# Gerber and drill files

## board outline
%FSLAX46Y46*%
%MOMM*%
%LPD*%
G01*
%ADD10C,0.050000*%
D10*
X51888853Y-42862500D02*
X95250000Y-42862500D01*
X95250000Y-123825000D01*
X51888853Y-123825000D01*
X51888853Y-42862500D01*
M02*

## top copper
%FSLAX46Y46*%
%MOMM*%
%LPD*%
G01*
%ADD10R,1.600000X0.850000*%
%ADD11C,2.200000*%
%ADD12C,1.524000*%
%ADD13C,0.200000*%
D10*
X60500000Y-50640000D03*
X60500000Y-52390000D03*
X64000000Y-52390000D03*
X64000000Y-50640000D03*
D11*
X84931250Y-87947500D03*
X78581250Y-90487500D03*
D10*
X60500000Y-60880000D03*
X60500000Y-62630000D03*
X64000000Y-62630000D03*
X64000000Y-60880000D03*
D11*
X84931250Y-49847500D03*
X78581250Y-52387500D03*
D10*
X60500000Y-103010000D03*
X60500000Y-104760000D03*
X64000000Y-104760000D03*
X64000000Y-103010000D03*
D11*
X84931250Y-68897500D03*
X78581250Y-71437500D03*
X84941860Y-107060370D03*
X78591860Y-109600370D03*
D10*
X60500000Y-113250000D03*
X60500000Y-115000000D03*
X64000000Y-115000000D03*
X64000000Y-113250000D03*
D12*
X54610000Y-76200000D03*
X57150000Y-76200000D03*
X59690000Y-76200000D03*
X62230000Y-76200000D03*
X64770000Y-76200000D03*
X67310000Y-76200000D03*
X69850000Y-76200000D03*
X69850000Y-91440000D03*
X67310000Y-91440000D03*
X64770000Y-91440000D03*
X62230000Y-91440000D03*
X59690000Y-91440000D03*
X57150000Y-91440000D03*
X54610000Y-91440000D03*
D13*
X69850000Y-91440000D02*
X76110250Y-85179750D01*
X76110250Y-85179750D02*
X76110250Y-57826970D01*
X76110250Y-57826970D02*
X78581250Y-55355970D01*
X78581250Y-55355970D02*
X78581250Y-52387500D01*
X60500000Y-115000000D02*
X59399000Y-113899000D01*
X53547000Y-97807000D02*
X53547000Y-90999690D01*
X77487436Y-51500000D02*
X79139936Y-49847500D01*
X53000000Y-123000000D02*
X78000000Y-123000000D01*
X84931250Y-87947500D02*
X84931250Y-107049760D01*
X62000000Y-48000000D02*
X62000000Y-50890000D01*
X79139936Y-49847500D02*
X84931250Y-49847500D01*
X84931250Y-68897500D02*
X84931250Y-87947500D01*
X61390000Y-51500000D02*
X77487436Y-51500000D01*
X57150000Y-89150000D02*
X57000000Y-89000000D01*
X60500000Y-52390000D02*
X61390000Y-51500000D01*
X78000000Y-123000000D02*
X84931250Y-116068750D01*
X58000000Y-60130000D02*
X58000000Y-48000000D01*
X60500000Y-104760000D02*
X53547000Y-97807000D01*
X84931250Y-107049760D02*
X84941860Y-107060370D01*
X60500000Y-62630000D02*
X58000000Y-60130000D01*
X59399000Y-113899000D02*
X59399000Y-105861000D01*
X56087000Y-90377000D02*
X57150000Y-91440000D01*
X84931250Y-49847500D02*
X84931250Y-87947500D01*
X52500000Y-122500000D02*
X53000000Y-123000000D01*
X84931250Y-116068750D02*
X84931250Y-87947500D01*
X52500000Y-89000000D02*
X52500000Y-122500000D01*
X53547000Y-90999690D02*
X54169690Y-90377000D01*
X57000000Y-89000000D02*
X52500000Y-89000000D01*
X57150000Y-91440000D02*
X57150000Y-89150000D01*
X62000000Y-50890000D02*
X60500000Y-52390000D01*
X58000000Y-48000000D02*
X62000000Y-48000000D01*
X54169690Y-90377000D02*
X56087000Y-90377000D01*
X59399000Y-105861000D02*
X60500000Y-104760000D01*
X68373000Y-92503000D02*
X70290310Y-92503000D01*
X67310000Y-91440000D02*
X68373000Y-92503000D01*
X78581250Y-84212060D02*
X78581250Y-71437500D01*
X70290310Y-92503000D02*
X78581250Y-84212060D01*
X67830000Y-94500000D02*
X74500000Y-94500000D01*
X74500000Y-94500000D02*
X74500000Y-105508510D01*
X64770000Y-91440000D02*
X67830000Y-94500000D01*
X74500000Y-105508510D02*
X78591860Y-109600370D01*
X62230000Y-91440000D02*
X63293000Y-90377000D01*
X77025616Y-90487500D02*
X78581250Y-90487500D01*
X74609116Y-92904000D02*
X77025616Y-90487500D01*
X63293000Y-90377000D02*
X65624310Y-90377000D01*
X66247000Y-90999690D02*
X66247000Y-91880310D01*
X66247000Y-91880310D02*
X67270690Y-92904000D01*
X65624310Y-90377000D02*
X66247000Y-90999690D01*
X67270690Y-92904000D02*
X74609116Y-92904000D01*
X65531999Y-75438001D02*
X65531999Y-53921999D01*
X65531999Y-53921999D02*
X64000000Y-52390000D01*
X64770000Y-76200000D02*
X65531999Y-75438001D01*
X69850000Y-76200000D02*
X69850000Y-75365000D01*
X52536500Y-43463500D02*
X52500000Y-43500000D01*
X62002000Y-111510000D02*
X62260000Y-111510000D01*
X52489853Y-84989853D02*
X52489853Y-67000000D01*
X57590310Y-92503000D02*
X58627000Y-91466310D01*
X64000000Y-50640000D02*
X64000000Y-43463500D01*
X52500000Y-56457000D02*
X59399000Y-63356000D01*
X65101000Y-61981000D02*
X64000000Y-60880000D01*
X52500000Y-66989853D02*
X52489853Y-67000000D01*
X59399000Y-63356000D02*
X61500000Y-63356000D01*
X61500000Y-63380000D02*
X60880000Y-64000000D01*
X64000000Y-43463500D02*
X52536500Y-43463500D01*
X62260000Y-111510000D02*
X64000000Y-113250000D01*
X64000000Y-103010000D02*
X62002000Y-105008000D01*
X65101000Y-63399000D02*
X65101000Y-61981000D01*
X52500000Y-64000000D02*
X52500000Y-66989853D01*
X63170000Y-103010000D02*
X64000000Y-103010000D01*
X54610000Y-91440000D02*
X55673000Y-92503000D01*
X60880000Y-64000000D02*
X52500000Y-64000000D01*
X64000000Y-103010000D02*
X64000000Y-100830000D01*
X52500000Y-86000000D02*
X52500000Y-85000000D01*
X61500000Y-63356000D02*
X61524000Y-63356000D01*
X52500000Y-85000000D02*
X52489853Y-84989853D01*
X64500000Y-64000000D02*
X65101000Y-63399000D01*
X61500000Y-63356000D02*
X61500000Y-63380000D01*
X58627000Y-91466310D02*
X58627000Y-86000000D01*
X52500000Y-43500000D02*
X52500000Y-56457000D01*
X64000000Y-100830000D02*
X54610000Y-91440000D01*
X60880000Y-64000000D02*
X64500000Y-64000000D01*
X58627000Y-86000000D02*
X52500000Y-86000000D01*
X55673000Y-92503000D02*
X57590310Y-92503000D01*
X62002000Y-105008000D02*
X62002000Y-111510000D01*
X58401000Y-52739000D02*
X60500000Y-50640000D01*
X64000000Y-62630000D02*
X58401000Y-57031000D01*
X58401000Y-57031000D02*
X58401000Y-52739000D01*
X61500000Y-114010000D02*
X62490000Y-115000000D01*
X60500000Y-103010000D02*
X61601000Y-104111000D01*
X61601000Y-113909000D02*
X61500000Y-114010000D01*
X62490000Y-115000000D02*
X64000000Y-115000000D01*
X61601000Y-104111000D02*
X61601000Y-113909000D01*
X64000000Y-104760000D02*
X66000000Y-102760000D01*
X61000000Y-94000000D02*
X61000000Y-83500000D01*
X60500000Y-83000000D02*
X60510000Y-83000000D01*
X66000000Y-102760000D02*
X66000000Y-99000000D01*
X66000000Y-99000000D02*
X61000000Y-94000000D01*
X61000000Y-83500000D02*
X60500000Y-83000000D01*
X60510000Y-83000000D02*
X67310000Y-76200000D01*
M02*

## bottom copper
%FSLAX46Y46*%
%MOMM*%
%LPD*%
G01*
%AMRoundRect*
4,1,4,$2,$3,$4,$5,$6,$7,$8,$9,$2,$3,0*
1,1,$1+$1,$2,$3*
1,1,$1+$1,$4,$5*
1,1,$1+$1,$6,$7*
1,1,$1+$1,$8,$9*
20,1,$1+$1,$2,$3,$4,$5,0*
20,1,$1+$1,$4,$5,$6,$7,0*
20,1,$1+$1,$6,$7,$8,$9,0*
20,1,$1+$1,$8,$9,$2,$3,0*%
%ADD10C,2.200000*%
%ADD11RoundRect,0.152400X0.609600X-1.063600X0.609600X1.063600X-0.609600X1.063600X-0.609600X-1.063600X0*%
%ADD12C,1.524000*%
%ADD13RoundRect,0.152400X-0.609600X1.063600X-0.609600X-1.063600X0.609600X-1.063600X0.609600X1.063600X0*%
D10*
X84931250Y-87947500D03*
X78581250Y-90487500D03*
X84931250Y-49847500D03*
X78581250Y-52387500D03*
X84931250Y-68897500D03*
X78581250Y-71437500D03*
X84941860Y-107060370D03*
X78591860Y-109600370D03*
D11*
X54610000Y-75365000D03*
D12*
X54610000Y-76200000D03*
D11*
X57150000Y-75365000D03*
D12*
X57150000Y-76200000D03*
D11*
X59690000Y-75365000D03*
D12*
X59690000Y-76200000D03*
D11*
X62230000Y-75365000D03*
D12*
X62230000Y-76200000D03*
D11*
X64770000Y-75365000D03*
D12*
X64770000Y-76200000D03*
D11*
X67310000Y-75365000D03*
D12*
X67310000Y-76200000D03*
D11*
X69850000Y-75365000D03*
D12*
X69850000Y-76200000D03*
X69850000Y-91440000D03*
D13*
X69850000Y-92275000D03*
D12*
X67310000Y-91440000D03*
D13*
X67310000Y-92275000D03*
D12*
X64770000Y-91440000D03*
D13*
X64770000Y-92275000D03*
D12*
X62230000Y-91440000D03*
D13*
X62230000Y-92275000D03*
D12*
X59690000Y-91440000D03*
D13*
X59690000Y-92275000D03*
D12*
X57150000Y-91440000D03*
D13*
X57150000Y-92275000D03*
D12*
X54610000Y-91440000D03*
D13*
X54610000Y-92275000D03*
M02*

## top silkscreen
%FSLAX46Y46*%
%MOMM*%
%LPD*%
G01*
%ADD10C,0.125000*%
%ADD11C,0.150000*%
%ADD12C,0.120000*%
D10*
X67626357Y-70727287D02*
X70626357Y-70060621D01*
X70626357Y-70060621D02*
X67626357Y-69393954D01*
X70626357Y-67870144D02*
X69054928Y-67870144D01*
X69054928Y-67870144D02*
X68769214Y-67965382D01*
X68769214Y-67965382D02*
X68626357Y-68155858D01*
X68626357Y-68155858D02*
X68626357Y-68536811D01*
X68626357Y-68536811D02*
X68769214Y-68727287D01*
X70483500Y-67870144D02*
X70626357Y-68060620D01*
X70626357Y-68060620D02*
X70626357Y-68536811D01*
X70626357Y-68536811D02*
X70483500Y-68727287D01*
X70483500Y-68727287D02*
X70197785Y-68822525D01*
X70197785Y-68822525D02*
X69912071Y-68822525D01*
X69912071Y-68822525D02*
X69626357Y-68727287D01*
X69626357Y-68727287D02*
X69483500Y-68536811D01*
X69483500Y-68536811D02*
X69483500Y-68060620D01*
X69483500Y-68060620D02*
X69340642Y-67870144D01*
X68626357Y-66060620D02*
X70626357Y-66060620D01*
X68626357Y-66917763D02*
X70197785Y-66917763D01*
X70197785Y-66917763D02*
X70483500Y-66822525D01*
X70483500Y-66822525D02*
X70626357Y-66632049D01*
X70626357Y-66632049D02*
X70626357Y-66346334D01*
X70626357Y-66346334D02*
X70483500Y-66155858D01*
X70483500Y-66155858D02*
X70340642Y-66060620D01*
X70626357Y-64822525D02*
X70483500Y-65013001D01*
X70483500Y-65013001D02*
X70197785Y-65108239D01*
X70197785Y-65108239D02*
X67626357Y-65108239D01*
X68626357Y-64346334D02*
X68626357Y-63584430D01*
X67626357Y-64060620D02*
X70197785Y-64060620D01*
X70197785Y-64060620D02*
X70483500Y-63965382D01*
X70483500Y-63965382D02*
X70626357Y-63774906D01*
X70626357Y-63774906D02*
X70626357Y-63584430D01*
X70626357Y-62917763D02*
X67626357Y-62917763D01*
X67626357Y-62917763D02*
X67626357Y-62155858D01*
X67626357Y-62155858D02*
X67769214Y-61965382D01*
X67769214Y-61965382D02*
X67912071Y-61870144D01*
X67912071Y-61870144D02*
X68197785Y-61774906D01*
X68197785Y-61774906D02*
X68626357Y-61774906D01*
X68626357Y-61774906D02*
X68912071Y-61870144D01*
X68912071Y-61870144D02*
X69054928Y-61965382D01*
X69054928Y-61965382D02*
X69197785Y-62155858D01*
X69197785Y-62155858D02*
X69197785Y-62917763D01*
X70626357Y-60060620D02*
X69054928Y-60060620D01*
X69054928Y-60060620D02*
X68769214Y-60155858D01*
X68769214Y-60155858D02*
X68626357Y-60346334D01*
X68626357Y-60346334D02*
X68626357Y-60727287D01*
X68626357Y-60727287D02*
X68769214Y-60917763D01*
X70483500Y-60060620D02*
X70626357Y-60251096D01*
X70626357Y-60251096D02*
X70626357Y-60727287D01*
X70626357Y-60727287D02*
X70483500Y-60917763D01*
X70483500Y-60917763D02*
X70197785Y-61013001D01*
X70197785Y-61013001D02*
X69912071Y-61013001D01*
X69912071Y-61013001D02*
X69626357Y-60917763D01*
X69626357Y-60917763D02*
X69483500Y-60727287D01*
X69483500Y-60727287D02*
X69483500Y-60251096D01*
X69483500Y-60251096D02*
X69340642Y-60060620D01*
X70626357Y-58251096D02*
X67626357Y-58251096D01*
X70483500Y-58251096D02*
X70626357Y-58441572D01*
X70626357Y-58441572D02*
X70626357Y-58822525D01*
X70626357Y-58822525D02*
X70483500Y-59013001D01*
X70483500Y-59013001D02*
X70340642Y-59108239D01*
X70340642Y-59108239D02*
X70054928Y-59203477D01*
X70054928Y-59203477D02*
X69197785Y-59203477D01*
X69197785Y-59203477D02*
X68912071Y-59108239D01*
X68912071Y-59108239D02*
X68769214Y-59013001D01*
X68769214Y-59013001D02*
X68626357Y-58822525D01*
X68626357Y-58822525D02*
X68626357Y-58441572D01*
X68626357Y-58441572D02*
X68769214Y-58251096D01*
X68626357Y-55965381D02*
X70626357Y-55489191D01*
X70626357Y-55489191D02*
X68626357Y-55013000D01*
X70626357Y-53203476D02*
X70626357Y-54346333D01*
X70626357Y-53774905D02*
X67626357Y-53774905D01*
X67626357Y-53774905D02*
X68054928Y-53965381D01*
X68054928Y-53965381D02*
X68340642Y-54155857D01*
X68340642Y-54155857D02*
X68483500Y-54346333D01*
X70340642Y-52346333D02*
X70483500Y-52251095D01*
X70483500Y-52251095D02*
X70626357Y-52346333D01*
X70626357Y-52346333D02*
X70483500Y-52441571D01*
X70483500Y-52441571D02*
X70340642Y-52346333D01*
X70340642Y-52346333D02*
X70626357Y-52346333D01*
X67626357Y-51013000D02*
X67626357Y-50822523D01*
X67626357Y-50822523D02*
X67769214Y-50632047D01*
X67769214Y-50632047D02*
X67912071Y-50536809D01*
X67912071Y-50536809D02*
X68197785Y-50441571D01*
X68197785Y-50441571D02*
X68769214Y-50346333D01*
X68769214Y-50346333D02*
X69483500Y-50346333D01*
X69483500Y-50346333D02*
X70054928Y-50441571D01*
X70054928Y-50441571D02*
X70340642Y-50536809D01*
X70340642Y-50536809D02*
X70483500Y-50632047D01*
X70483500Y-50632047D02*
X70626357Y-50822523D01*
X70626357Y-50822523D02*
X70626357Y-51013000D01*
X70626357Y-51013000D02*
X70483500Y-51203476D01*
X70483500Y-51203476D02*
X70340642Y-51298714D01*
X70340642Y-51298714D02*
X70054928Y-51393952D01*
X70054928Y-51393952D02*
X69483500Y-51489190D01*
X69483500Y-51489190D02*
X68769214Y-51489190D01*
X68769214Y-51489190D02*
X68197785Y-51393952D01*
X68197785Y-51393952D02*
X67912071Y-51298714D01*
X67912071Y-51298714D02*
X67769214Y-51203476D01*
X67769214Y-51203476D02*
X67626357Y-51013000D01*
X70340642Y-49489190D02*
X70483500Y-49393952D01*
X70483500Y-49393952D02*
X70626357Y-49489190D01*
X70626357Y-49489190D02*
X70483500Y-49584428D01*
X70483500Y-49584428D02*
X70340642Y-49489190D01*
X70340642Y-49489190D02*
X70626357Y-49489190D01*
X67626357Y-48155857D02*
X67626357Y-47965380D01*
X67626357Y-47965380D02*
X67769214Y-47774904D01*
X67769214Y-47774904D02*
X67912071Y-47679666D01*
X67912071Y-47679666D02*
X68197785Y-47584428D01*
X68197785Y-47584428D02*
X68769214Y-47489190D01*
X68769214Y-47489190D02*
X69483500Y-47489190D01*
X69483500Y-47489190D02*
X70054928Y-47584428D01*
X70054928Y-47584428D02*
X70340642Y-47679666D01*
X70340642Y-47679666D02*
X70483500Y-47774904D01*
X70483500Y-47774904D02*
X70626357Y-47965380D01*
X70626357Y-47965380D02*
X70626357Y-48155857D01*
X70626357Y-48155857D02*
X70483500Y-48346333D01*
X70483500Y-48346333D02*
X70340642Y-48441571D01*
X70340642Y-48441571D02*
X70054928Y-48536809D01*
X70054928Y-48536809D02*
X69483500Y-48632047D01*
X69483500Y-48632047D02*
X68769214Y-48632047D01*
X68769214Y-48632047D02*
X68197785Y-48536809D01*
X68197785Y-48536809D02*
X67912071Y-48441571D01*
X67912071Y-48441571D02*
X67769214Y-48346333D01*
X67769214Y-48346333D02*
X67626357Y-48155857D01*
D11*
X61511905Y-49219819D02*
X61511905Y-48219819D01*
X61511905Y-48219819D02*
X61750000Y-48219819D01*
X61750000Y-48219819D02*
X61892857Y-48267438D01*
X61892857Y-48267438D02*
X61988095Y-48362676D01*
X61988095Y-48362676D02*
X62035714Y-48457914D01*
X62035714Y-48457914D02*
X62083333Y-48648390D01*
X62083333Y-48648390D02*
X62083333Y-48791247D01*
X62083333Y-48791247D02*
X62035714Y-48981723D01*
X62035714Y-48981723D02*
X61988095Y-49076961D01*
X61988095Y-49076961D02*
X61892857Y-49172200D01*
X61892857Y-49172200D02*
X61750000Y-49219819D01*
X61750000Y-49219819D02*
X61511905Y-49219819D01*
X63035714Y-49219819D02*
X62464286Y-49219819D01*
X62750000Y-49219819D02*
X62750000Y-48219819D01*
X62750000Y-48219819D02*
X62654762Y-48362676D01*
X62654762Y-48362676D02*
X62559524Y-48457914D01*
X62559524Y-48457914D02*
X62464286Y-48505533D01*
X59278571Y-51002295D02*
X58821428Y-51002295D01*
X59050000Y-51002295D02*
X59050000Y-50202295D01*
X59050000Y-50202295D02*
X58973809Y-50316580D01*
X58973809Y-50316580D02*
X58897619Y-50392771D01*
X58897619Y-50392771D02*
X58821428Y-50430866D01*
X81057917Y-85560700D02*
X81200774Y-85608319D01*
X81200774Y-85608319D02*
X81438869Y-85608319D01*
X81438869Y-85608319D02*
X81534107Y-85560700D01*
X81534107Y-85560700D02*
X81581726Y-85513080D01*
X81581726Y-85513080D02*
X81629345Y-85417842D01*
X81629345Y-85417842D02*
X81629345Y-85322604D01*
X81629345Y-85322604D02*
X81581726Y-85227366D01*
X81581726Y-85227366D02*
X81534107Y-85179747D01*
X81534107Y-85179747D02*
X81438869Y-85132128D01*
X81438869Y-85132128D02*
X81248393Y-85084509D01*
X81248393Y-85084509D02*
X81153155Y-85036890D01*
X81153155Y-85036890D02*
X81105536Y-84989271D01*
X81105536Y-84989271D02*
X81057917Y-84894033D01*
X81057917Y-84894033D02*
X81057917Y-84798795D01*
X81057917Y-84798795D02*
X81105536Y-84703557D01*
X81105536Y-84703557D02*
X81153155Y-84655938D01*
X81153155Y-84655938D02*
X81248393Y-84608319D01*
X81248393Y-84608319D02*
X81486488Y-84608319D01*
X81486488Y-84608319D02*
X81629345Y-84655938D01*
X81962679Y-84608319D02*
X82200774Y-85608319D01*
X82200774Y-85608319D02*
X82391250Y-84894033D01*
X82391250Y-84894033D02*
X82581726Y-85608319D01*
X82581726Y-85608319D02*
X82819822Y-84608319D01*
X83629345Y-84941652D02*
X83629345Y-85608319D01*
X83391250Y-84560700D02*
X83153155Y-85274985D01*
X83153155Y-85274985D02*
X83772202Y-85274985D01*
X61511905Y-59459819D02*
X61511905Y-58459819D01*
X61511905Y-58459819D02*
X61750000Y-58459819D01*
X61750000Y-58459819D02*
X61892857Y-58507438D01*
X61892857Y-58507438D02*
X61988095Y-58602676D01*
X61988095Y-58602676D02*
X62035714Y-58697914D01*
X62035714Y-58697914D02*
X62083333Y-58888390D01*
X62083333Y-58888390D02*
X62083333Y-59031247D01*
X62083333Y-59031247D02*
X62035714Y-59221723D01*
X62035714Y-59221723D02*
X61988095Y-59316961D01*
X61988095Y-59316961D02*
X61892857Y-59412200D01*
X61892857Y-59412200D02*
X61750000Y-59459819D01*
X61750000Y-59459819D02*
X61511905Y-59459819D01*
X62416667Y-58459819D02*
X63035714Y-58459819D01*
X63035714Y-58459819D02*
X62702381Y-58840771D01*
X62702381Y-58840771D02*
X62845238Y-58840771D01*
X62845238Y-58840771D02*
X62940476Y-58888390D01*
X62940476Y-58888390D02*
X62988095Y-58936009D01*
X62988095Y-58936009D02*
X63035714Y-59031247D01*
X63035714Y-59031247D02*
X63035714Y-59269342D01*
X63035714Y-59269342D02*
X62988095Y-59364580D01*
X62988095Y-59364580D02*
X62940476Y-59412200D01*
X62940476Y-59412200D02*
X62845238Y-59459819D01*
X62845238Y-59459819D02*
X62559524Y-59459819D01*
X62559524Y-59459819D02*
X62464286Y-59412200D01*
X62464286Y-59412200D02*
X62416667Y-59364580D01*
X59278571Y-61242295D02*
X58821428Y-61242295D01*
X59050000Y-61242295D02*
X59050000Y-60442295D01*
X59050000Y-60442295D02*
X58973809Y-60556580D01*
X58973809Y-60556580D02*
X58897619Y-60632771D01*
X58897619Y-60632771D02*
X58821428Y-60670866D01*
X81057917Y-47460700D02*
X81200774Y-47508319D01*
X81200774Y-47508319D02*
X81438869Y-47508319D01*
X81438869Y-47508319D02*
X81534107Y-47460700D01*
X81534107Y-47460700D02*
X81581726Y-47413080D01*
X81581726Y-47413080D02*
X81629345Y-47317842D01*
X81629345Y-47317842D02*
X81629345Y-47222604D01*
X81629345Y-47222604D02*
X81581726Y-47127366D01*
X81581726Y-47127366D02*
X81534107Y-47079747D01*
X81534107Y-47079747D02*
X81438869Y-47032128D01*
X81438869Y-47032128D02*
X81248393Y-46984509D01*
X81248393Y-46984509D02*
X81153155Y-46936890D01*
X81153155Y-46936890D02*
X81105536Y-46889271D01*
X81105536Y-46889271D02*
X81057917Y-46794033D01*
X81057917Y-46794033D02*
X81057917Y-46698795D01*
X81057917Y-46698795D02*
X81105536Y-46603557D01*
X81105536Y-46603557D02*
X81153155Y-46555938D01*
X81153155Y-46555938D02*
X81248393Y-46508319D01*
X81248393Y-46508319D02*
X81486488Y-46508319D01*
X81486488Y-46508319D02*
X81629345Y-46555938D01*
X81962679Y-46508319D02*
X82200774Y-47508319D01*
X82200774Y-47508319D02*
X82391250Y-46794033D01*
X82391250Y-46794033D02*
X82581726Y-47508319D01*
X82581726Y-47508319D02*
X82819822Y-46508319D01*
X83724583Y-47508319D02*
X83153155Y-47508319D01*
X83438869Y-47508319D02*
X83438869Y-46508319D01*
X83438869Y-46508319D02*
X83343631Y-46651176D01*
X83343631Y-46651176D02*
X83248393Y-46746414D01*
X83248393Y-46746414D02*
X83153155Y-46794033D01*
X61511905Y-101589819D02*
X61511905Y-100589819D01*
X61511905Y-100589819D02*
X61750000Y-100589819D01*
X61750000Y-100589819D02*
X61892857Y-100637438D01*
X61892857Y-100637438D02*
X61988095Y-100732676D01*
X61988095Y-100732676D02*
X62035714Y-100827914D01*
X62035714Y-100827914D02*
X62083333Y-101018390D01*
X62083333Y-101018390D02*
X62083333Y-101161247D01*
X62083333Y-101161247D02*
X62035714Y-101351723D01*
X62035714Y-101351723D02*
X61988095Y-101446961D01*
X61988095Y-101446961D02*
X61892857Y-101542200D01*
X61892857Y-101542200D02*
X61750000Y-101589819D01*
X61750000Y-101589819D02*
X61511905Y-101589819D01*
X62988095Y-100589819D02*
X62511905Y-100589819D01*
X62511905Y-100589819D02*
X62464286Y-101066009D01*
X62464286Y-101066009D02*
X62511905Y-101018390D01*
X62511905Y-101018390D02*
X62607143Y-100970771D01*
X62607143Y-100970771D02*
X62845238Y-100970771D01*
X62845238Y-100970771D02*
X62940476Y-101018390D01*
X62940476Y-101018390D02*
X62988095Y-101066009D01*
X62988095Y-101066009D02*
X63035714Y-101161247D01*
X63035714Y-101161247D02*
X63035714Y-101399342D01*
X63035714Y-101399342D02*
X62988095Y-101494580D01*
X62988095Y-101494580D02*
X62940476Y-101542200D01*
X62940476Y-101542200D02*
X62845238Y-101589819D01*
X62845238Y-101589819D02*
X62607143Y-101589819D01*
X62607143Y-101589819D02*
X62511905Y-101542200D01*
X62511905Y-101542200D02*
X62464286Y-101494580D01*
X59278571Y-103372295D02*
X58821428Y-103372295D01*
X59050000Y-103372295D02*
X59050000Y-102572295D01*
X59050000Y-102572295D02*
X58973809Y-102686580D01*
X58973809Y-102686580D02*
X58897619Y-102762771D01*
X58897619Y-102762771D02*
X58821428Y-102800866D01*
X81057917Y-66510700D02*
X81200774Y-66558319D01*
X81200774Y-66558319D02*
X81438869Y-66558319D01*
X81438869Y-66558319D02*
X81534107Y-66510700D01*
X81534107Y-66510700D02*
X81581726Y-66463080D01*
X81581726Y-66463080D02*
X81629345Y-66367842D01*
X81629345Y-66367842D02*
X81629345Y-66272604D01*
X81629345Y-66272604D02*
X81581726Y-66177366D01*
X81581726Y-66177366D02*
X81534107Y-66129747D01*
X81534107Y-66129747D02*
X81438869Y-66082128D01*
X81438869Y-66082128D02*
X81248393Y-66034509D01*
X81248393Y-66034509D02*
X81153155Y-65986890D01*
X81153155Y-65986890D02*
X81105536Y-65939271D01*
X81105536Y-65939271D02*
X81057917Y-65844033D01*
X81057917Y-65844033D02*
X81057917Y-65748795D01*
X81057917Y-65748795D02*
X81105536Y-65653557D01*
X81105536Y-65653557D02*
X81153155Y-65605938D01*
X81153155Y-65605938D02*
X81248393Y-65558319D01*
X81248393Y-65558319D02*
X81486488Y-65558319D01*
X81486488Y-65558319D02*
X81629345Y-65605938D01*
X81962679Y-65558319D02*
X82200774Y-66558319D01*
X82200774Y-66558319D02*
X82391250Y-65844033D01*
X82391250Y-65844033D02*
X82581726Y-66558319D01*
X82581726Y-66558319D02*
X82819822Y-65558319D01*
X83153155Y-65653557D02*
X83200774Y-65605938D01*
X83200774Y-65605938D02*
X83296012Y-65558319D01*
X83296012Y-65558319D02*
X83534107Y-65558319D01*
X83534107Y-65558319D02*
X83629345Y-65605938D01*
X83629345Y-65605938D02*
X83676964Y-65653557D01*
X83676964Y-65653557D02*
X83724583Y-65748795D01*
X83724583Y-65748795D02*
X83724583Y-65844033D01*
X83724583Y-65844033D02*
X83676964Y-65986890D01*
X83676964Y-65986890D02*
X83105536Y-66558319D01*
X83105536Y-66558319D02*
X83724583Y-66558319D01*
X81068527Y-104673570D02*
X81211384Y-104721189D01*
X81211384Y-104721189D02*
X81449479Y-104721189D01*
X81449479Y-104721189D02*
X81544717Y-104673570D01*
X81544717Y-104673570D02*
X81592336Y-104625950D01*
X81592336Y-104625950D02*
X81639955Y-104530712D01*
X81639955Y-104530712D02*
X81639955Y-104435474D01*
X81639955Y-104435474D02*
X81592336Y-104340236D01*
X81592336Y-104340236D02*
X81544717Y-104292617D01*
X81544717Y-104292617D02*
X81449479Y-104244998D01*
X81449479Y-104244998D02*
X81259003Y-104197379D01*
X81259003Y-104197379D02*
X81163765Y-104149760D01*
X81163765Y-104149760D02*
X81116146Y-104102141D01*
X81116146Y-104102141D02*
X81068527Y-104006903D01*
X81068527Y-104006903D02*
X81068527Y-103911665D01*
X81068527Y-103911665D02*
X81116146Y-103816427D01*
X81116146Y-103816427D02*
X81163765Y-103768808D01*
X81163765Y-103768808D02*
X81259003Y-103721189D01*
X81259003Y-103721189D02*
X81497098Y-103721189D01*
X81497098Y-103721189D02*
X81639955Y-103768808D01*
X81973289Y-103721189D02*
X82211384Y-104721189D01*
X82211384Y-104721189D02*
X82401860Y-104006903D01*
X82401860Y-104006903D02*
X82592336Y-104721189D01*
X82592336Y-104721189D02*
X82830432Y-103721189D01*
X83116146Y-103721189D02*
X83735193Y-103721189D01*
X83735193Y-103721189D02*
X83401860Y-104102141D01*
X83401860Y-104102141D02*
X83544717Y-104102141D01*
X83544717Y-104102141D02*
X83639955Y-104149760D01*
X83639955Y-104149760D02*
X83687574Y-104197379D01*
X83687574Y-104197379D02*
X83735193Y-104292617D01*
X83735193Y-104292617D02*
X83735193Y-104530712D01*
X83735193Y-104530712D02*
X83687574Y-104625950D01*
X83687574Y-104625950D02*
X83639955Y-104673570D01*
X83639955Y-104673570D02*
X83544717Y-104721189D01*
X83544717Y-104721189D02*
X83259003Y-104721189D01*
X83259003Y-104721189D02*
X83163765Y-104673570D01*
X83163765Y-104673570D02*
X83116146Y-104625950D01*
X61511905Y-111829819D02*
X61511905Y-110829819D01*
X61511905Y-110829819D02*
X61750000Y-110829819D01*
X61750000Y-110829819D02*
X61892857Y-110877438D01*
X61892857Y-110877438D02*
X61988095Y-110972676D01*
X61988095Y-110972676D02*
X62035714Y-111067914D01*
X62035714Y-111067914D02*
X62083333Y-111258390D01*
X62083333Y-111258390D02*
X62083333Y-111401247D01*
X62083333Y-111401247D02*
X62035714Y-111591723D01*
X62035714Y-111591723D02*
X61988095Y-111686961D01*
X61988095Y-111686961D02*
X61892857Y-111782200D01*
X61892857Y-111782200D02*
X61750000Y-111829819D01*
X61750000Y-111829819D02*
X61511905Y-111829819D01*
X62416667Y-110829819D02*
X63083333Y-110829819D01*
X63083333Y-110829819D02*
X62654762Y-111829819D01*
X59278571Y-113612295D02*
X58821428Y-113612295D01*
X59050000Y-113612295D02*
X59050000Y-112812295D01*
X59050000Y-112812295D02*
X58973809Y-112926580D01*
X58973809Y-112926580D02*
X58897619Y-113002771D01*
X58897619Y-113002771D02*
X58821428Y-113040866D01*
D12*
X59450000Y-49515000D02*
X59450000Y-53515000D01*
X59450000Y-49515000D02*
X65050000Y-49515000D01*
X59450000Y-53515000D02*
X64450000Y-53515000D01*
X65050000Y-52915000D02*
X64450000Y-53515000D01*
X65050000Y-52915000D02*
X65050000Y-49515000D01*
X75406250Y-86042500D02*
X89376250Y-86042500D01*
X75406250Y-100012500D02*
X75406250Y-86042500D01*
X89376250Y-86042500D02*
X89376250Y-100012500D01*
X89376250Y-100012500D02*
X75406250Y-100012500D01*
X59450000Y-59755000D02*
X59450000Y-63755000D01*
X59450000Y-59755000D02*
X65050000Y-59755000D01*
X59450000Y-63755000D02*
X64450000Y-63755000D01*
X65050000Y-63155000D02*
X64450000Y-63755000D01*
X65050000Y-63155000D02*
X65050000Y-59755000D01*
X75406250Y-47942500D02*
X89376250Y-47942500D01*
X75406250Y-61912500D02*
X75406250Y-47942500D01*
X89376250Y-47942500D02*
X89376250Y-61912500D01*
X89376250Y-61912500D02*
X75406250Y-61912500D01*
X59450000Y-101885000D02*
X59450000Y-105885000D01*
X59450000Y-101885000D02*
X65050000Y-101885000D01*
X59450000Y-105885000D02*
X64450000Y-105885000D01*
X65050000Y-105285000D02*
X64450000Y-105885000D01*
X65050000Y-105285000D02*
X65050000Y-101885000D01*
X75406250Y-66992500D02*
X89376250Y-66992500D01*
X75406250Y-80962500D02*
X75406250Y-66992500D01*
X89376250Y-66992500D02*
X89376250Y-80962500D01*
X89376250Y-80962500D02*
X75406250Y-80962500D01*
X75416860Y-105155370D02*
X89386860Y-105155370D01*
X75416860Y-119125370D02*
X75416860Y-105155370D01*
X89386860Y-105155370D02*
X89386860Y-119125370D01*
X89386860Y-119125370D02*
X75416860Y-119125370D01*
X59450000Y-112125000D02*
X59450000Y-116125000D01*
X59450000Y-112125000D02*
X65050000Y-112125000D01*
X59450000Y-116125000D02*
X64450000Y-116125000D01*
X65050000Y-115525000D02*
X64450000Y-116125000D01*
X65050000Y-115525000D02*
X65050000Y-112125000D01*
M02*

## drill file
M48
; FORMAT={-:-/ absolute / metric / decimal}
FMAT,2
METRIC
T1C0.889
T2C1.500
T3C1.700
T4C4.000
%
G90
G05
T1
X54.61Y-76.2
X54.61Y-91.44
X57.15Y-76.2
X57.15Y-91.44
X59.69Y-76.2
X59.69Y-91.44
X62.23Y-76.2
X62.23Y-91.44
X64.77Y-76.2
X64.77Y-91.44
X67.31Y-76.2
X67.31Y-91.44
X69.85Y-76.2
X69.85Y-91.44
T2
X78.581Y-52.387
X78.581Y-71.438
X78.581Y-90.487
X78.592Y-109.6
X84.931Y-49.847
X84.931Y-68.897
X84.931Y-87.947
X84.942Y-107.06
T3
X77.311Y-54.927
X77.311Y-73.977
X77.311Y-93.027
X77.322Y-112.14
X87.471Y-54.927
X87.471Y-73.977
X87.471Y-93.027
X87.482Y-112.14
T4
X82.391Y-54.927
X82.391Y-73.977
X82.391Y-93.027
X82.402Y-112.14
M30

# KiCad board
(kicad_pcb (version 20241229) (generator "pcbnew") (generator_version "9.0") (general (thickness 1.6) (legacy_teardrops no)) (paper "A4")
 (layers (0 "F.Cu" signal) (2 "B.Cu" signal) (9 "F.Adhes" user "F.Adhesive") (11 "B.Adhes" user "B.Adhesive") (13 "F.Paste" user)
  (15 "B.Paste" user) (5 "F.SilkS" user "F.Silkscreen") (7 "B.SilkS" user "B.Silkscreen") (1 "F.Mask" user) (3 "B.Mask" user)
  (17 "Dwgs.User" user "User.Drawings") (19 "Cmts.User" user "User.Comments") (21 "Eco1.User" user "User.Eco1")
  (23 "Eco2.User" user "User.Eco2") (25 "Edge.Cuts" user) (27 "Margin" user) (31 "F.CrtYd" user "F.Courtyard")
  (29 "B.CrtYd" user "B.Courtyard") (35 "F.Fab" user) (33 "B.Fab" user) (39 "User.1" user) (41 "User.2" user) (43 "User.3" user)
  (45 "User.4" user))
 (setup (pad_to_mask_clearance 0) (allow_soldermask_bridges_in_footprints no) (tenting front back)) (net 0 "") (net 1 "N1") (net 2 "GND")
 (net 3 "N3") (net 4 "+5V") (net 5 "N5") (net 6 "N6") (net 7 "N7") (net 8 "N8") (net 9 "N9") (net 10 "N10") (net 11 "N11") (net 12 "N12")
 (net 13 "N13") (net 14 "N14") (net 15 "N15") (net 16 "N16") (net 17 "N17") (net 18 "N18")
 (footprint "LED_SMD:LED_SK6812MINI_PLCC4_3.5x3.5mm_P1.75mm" (layer "F.Cu") (at 62.25 51.515)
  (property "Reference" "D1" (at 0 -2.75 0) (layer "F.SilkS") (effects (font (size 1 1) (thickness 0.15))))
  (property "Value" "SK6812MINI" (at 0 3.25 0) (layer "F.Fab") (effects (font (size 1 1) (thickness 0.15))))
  (fp_line (start -2.8 -2) (end -2.8 2) (stroke (width 0.12) (type default)) (layer "F.SilkS"))
  (fp_line (start -2.8 -2) (end 2.8 -2) (stroke (width 0.12) (type solid)) (layer "F.SilkS"))
  (fp_line (start -2.8 2) (end 2.2 2) (stroke (width 0.12) (type solid)) (layer "F.SilkS"))
  (fp_line (start 2.8 1.4) (end 2.2 2) (stroke (width 0.12) (type default)) (layer "F.SilkS"))
  (fp_line (start 2.8 1.4) (end 2.8 -2) (stroke (width 0.12) (type solid)) (layer "F.SilkS"))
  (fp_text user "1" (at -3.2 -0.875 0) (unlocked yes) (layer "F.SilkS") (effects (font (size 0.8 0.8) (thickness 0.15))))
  (pad "1" smd rect (at -1.75 -0.875) (size 1.6 0.85) (layers "F.Cu" "F.Mask" "F.Paste") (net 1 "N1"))
  (pad "2" smd rect (at -1.75 0.875) (size 1.6 0.85) (layers "F.Cu" "F.Mask" "F.Paste") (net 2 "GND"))
  (pad "3" smd rect (at 1.75 0.875) (size 1.6 0.85) (layers "F.Cu" "F.Mask" "F.Paste") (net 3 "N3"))
  (pad "4" smd rect (at 1.75 -0.875) (size 1.6 0.85) (layers "F.Cu" "F.Mask" "F.Paste") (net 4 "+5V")))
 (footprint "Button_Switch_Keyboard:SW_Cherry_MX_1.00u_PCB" (layer "F.Cu") (at 84.93125 87.9475)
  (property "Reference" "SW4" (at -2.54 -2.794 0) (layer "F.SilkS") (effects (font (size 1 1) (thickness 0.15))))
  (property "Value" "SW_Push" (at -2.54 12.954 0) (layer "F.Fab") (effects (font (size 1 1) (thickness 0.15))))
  (fp_line (start -9.525 -1.905) (end 4.445 -1.905) (stroke (width 0.12) (type solid)) (layer "F.SilkS"))
  (fp_line (start -9.525 12.065) (end -9.525 -1.905) (stroke (width 0.12) (type solid)) (layer "F.SilkS"))
  (fp_line (start 4.445 -1.905) (end 4.445 12.065) (stroke (width 0.12) (type solid)) (layer "F.SilkS"))
  (fp_line (start 4.445 12.065) (end -9.525 12.065) (stroke (width 0.12) (type solid)) (layer "F.SilkS"))
  (pad "" np_thru_hole circle (at -7.62 5.08) (size 1.7 1.7) (drill 1.7) (layers "*.Cu" "*.Mask"))
  (pad "" np_thru_hole circle (at -2.54 5.08) (size 4 4) (drill 4) (layers "*.Cu" "*.Mask"))
  (pad "" np_thru_hole circle (at 2.54 5.08) (size 1.7 1.7) (drill 1.7) (layers "*.Cu" "*.Mask"))
  (pad "1" thru_hole circle (at 0 0) (size 2.2 2.2) (drill 1.5) (layers "*.Cu" "*.Mask") (remove_unused_layers no) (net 2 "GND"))
  (pad "2" thru_hole circle (at -6.35 2.54) (size 2.2 2.2) (drill 1.5) (layers "*.Cu" "*.Mask") (remove_unused_layers no) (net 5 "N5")))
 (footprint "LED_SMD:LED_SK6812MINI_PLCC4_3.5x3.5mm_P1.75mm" (layer "F.Cu") (at 62.25 61.755)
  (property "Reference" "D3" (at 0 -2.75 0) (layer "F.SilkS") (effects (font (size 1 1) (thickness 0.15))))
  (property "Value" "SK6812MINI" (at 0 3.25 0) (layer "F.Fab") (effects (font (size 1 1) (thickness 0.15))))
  (fp_line (start -2.8 -2) (end -2.8 2) (stroke (width 0.12) (type default)) (layer "F.SilkS"))
  (fp_line (start -2.8 -2) (end 2.8 -2) (stroke (width 0.12) (type solid)) (layer "F.SilkS"))
  (fp_line (start -2.8 2) (end 2.2 2) (stroke (width 0.12) (type solid)) (layer "F.SilkS"))
  (fp_line (start 2.8 1.4) (end 2.2 2) (stroke (width 0.12) (type default)) (layer "F.SilkS"))
  (fp_line (start 2.8 1.4) (end 2.8 -2) (stroke (width 0.12) (type solid)) (layer "F.SilkS"))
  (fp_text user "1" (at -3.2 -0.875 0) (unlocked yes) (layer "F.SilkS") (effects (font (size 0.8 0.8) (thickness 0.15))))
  (pad "1" smd rect (at -1.75 -0.875) (size 1.6 0.85) (layers "F.Cu" "F.Mask" "F.Paste") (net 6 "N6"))
  (pad "2" smd rect (at -1.75 0.875) (size 1.6 0.85) (layers "F.Cu" "F.Mask" "F.Paste") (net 2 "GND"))
  (pad "3" smd rect (at 1.75 0.875) (size 1.6 0.85) (layers "F.Cu" "F.Mask" "F.Paste") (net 1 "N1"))
  (pad "4" smd rect (at 1.75 -0.875) (size 1.6 0.85) (layers "F.Cu" "F.Mask" "F.Paste") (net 4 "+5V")))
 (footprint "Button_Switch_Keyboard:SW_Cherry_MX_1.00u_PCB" (layer "F.Cu") (at 84.93125 49.8475)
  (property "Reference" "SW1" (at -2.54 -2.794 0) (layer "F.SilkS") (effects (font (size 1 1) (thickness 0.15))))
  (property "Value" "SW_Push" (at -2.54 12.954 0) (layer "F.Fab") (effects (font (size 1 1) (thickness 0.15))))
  (fp_line (start -9.525 -1.905) (end 4.445 -1.905) (stroke (width 0.12) (type solid)) (layer "F.SilkS"))
  (fp_line (start -9.525 12.065) (end -9.525 -1.905) (stroke (width 0.12) (type solid)) (layer "F.SilkS"))
  (fp_line (start 4.445 -1.905) (end 4.445 12.065) (stroke (width 0.12) (type solid)) (layer "F.SilkS"))
  (fp_line (start 4.445 12.065) (end -9.525 12.065) (stroke (width 0.12) (type solid)) (layer "F.SilkS"))
  (pad "" np_thru_hole circle (at -7.62 5.08) (size 1.7 1.7) (drill 1.7) (layers "*.Cu" "*.Mask"))
  (pad "" np_thru_hole circle (at -2.54 5.08) (size 4 4) (drill 4) (layers "*.Cu" "*.Mask"))
  (pad "" np_thru_hole circle (at 2.54 5.08) (size 1.7 1.7) (drill 1.7) (layers "*.Cu" "*.Mask"))
  (pad "1" thru_hole circle (at 0 0) (size 2.2 2.2) (drill 1.5) (layers "*.Cu" "*.Mask") (remove_unused_layers no) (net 2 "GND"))
  (pad "2" thru_hole circle (at -6.35 2.54) (size 2.2 2.2) (drill 1.5) (layers "*.Cu" "*.Mask") (remove_unused_layers no) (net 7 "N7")))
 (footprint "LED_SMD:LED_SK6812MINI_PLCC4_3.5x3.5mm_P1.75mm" (layer "F.Cu") (at 62.25 103.885)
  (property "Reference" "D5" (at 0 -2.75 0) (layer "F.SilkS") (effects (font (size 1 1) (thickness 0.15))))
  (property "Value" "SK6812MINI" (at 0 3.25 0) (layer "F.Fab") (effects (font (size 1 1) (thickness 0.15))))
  (fp_line (start -2.8 -2) (end -2.8 2) (stroke (width 0.12) (type default)) (layer "F.SilkS"))
  (fp_line (start -2.8 -2) (end 2.8 -2) (stroke (width 0.12) (type solid)) (layer "F.SilkS"))
  (fp_line (start -2.8 2) (end 2.2 2) (stroke (width 0.12) (type solid)) (layer "F.SilkS"))
  (fp_line (start 2.8 1.4) (end 2.2 2) (stroke (width 0.12) (type default)) (layer "F.SilkS"))
  (fp_line (start 2.8 1.4) (end 2.8 -2) (stroke (width 0.12) (type solid)) (layer "F.SilkS"))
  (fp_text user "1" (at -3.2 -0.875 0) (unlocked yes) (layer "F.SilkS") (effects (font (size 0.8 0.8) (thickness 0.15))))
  (pad "1" smd rect (at -1.75 -0.875) (size 1.6 0.85) (layers "F.Cu" "F.Mask" "F.Paste") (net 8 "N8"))
  (pad "2" smd rect (at -1.75 0.875) (size 1.6 0.85) (layers "F.Cu" "F.Mask" "F.Paste") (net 2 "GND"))
  (pad "3" smd rect (at 1.75 0.875) (size 1.6 0.85) (layers "F.Cu" "F.Mask" "F.Paste") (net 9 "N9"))
  (pad "4" smd rect (at 1.75 -0.875) (size 1.6 0.85) (layers "F.Cu" "F.Mask" "F.Paste") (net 4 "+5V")))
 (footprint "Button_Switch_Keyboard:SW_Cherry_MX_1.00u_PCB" (layer "F.Cu") (at 84.93125 68.8975)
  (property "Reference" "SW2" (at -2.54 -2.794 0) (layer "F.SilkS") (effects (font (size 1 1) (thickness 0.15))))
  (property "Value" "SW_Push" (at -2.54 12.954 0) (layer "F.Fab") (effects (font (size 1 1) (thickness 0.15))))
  (fp_line (start -9.525 -1.905) (end 4.445 -1.905) (stroke (width 0.12) (type solid)) (layer "F.SilkS"))
  (fp_line (start -9.525 12.065) (end -9.525 -1.905) (stroke (width 0.12) (type solid)) (layer "F.SilkS"))
  (fp_line (start 4.445 -1.905) (end 4.445 12.065) (stroke (width 0.12) (type solid)) (layer "F.SilkS"))
  (fp_line (start 4.445 12.065) (end -9.525 12.065) (stroke (width 0.12) (type solid)) (layer "F.SilkS"))
  (pad "" np_thru_hole circle (at -7.62 5.08) (size 1.7 1.7) (drill 1.7) (layers "*.Cu" "*.Mask"))
  (pad "" np_thru_hole circle (at -2.54 5.08) (size 4 4) (drill 4) (layers "*.Cu" "*.Mask"))
  (pad "" np_thru_hole circle (at 2.54 5.08) (size 1.7 1.7) (drill 1.7) (layers "*.Cu" "*.Mask"))
  (pad "1" thru_hole circle (at 0 0) (size 2.2 2.2) (drill 1.5) (layers "*.Cu" "*.Mask") (remove_unused_layers no) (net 2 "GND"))
  (pad "2" thru_hole circle (at -6.35 2.54) (size 2.2 2.2) (drill 1.5) (layers "*.Cu" "*.Mask") (remove_unused_layers no) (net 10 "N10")))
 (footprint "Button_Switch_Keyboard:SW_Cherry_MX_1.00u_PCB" (layer "F.Cu") (at 84.94186 107.06037)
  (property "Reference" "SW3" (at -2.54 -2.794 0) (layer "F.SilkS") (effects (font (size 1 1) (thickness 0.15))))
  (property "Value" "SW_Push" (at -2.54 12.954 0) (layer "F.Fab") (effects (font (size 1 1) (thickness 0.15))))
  (fp_line (start -9.525 -1.905) (end 4.445 -1.905) (stroke (width 0.12) (type solid)) (layer "F.SilkS"))
  (fp_line (start -9.525 12.065) (end -9.525 -1.905) (stroke (width 0.12) (type solid)) (layer "F.SilkS"))
  (fp_line (start 4.445 -1.905) (end 4.445 12.065) (stroke (width 0.12) (type solid)) (layer "F.SilkS"))
  (fp_line (start 4.445 12.065) (end -9.525 12.065) (stroke (width 0.12) (type solid)) (layer "F.SilkS"))
  (pad "" np_thru_hole circle (at -7.62 5.08) (size 1.7 1.7) (drill 1.7) (layers "*.Cu" "*.Mask"))
  (pad "" np_thru_hole circle (at -2.54 5.08) (size 4 4) (drill 4) (layers "*.Cu" "*.Mask"))
  (pad "" np_thru_hole circle (at 2.54 5.08) (size 1.7 1.7) (drill 1.7) (layers "*.Cu" "*.Mask"))
  (pad "1" thru_hole circle (at 0 0) (size 2.2 2.2) (drill 1.5) (layers "*.Cu" "*.Mask") (remove_unused_layers no) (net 2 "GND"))
  (pad "2" thru_hole circle (at -6.35 2.54) (size 2.2 2.2) (drill 1.5) (layers "*.Cu" "*.Mask") (remove_unused_layers no) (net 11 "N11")))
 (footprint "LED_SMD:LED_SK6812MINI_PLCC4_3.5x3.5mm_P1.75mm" (layer "F.Cu") (at 62.25 114.125)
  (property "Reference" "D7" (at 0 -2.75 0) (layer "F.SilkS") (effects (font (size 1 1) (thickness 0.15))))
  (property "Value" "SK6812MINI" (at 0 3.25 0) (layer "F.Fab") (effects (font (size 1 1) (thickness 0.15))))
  (fp_line (start -2.8 -2) (end -2.8 2) (stroke (width 0.12) (type default)) (layer "F.SilkS"))
  (fp_line (start -2.8 -2) (end 2.8 -2) (stroke (width 0.12) (type solid)) (layer "F.SilkS"))
  (fp_line (start -2.8 2) (end 2.2 2) (stroke (width 0.12) (type solid)) (layer "F.SilkS"))
  (fp_line (start 2.8 1.4) (end 2.2 2) (stroke (width 0.12) (type default)) (layer "F.SilkS"))
  (fp_line (start 2.8 1.4) (end 2.8 -2) (stroke (width 0.12) (type solid)) (layer "F.SilkS"))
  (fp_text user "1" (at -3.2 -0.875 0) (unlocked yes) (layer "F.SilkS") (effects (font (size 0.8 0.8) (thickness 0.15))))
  (pad "1" smd rect (at -1.75 -0.875) (size 1.6 0.85) (layers "F.Cu" "F.Mask" "F.Paste") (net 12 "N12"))
  (pad "2" smd rect (at -1.75 0.875) (size 1.6 0.85) (layers "F.Cu" "F.Mask" "F.Paste") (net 2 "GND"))
  (pad "3" smd rect (at 1.75 0.875) (size 1.6 0.85) (layers "F.Cu" "F.Mask" "F.Paste") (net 8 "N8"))
  (pad "4" smd rect (at 1.75 -0.875) (size 1.6 0.85) (layers "F.Cu" "F.Mask" "F.Paste") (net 4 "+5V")))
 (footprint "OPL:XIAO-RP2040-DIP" (layer "B.Cu") (at 62.23 83.82 -90)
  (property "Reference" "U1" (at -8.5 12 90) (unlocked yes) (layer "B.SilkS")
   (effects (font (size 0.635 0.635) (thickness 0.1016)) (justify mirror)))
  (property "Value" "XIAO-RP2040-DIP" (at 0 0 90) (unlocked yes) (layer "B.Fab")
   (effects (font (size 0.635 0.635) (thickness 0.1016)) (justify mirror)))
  (pad "1" smd roundrect (at -8.455 7.62 90) (size 2.432 1.524) (layers "B.Cu" "B.Mask") (roundrect_rratio 0.1) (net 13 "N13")
   (thermal_bridge_angle 45))
  (pad "1" thru_hole circle (at -7.62 7.62 90) (size 1.524 1.524) (drill 0.889) (layers "*.Cu" "*.Mask") (remove_unused_layers no)
   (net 13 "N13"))
  (pad "2" smd roundrect (at -8.455 5.08 90) (size 2.432 1.524) (layers "B.Cu" "B.Mask") (roundrect_rratio 0.1) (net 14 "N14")
   (thermal_bridge_angle 45))
  (pad "2" thru_hole circle (at -7.62 5.08 90) (size 1.524 1.524) (drill 0.889) (layers "*.Cu" "*.Mask") (remove_unused_layers no)
   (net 14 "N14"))
  (pad "3" smd roundrect (at -8.455 2.54 90) (size 2.432 1.524) (layers "B.Cu" "B.Mask") (roundrect_rratio 0.1) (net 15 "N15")
   (thermal_bridge_angle 45))
  (pad "3" thru_hole circle (at -7.62 2.54 90) (size 1.524 1.524) (drill 0.889) (layers "*.Cu" "*.Mask") (remove_unused_layers no)
   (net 15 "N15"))
  (pad "4" smd roundrect (at -8.455 0 90) (size 2.432 1.524) (layers "B.Cu" "B.Mask") (roundrect_rratio 0.1) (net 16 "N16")
   (thermal_bridge_angle 45))
  (pad "4" thru_hole circle (at -7.62 0 90) (size 1.524 1.524) (drill 0.889) (layers "*.Cu" "*.Mask") (remove_unused_layers no)
   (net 16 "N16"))
  (pad "5" smd roundrect (at -8.455 -2.54 90) (size 2.432 1.524) (layers "B.Cu" "B.Mask") (roundrect_rratio 0.1) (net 3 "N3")
   (thermal_bridge_angle 45))
  (pad "5" thru_hole circle (at -7.62 -2.54 90) (size 1.524 1.524) (drill 0.889) (layers "*.Cu" "*.Mask") (remove_unused_layers no)
   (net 3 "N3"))
  (pad "6" smd roundrect (at -8.455 -5.08 90) (size 2.432 1.524) (layers "B.Cu" "B.Mask") (roundrect_rratio 0.1) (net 9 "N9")
   (thermal_bridge_angle 45))
  (pad "6" thru_hole circle (at -7.62 -5.08 90) (size 1.524 1.524) (drill 0.889) (layers "*.Cu" "*.Mask") (remove_unused_layers no)
   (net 9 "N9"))
  (pad "7" smd roundrect (at -8.455 -7.62 90) (size 2.432 1.524) (layers "B.Cu" "B.Mask") (roundrect_rratio 0.1) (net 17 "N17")
   (thermal_bridge_angle 45))
  (pad "7" thru_hole circle (at -7.62 -7.62 90) (size 1.524 1.524) (drill 0.889) (layers "*.Cu" "*.Mask") (remove_unused_layers no)
   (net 17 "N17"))
  (pad "8" thru_hole circle (at 7.62 -7.62 270) (size 1.524 1.524) (drill 0.889) (layers "*.Cu" "*.Mask") (remove_unused_layers no)
   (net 7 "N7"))
  (pad "8" smd roundrect (at 8.455 -7.62 270) (size 2.432 1.524) (layers "B.Cu" "B.Mask") (roundrect_rratio 0.1) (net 7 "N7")
   (thermal_bridge_angle 45))
  (pad "9" thru_hole circle (at 7.62 -5.08 270) (size 1.524 1.524) (drill 0.889) (layers "*.Cu" "*.Mask") (remove_unused_layers no)
   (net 10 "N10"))
  (pad "9" smd roundrect (at 8.455 -5.08 270) (size 2.432 1.524) (layers "B.Cu" "B.Mask") (roundrect_rratio 0.1) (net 10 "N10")
   (thermal_bridge_angle 45))
  (pad "10" thru_hole circle (at 7.62 -2.54 270) (size 1.524 1.524) (drill 0.889) (layers "*.Cu" "*.Mask") (remove_unused_layers no)
   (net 11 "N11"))
  (pad "10" smd roundrect (at 8.455 -2.54 270) (size 2.432 1.524) (layers "B.Cu" "B.Mask") (roundrect_rratio 0.1) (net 11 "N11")
   (thermal_bridge_angle 45))
  (pad "11" thru_hole circle (at 7.62 0 270) (size 1.524 1.524) (drill 0.889) (layers "*.Cu" "*.Mask") (remove_unused_layers no)
   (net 5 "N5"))
  (pad "11" smd roundrect (at 8.455 0 270) (size 2.432 1.524) (layers "B.Cu" "B.Mask") (roundrect_rratio 0.1) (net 5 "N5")
   (thermal_bridge_angle 45))
  (pad "12" thru_hole circle (at 7.62 2.54 270) (size 1.524 1.524) (drill 0.889) (layers "*.Cu" "*.Mask") (remove_unused_layers no)
   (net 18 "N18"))
  (pad "12" smd roundrect (at 8.455 2.54 270) (size 2.432 1.524) (layers "B.Cu" "B.Mask") (roundrect_rratio 0.1) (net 18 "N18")
   (thermal_bridge_angle 45))
  (pad "13" thru_hole circle (at 7.62 5.08 270) (size 1.524 1.524) (drill 0.889) (layers "*.Cu" "*.Mask") (remove_unused_layers no)
   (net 2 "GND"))
  (pad "13" smd roundrect (at 8.455 5.08 270) (size 2.432 1.524) (layers "B.Cu" "B.Mask") (roundrect_rratio 0.1) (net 2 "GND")
   (thermal_bridge_angle 45))
  (pad "14" thru_hole circle (at 7.62 7.62 270) (size 1.524 1.524) (drill 0.889) (layers "*.Cu" "*.Mask") (remove_unused_layers no)
   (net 4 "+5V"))
  (pad "14" smd roundrect (at 8.455 7.62 270) (size 2.432 1.524) (layers "B.Cu" "B.Mask") (roundrect_rratio 0.1) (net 4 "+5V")
   (thermal_bridge_angle 45)))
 (gr_rect (start 51.888853 42.8625) (end 95.25 123.825) (stroke (width 0.05) (type default)) (fill no) (layer "Edge.Cuts"))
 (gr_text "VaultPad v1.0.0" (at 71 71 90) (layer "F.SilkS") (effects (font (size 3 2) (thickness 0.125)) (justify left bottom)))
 (segment (start 69.85 91.44) (end 76.11025 85.17975) (width 0.2) (layer "F.Cu") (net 7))
 (segment (start 76.11025 85.17975) (end 76.11025 57.82697) (width 0.2) (layer "F.Cu") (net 7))
 (segment (start 76.11025 57.82697) (end 78.58125 55.35597) (width 0.2) (layer "F.Cu") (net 7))
 (segment (start 78.58125 55.35597) (end 78.58125 52.3875) (width 0.2) (layer "F.Cu") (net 7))
 (segment (start 60.5 115) (end 59.399 113.899) (width 0.2) (layer "F.Cu") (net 2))
 (segment (start 53.547 97.807) (end 53.547 90.99969) (width 0.2) (layer "F.Cu") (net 2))
 (segment (start 77.487436 51.5) (end 79.139936 49.8475) (width 0.2) (layer "F.Cu") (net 2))
 (segment (start 53 123) (end 78 123) (width 0.2) (layer "F.Cu") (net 2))
 (segment (start 84.93125 87.9475) (end 84.93125 107.04976) (width 0.2) (layer "F.Cu") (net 2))
 (segment (start 62 48) (end 62 50.89) (width 0.2) (layer "F.Cu") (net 2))
 (segment (start 79.139936 49.8475) (end 84.93125 49.8475) (width 0.2) (layer "F.Cu") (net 2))
 (segment (start 84.93125 68.8975) (end 84.93125 87.9475) (width 0.2) (layer "F.Cu") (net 2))
 (segment (start 61.39 51.5) (end 77.487436 51.5) (width 0.2) (layer "F.Cu") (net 2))
 (segment (start 57.15 89.15) (end 57 89) (width 0.2) (layer "F.Cu") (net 2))
 (segment (start 60.5 52.39) (end 61.39 51.5) (width 0.2) (layer "F.Cu") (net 2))
 (segment (start 78 123) (end 84.93125 116.06875) (width 0.2) (layer "F.Cu") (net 2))
 (segment (start 58 60.13) (end 58 48) (width 0.2) (layer "F.Cu") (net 2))
 (segment (start 60.5 104.76) (end 53.547 97.807) (width 0.2) (layer "F.Cu") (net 2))
 (segment (start 84.93125 107.04976) (end 84.94186 107.06037) (width 0.2) (layer "F.Cu") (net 2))
 (segment (start 60.5 62.63) (end 58 60.13) (width 0.2) (layer "F.Cu") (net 2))
 (segment (start 59.399 113.899) (end 59.399 105.861) (width 0.2) (layer "F.Cu") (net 2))
 (segment (start 56.087 90.377) (end 57.15 91.44) (width 0.2) (layer "F.Cu") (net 2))
 (segment (start 84.93125 49.8475) (end 84.93125 87.9475) (width 0.2) (layer "F.Cu") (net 2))
 (segment (start 52.5 122.5) (end 53 123) (width 0.2) (layer "F.Cu") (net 2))
 (segment (start 84.93125 116.06875) (end 84.93125 87.9475) (width 0.2) (layer "F.Cu") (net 2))
 (segment (start 52.5 89) (end 52.5 122.5) (width 0.2) (layer "F.Cu") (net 2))
 (segment (start 53.547 90.99969) (end 54.16969 90.377) (width 0.2) (layer "F.Cu") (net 2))
 (segment (start 57 89) (end 52.5 89) (width 0.2) (layer "F.Cu") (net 2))
 (segment (start 57.15 91.44) (end 57.15 89.15) (width 0.2) (layer "F.Cu") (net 2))
 (segment (start 62 50.89) (end 60.5 52.39) (width 0.2) (layer "F.Cu") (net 2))
 (segment (start 58 48) (end 62 48) (width 0.2) (layer "F.Cu") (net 2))
 (segment (start 54.16969 90.377) (end 56.087 90.377) (width 0.2) (layer "F.Cu") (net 2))
 (segment (start 59.399 105.861) (end 60.5 104.76) (width 0.2) (layer "F.Cu") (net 2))
 (segment (start 68.373 92.503) (end 70.29031 92.503) (width 0.2) (layer "F.Cu") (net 10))
 (segment (start 67.31 91.44) (end 68.373 92.503) (width 0.2) (layer "F.Cu") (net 10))
 (segment (start 78.58125 84.21206) (end 78.58125 71.4375) (width 0.2) (layer "F.Cu") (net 10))
 (segment (start 70.29031 92.503) (end 78.58125 84.21206) (width 0.2) (layer "F.Cu") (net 10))
 (segment (start 67.83 94.5) (end 74.5 94.5) (width 0.2) (layer "F.Cu") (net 11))
 (segment (start 74.5 94.5) (end 74.5 105.50851) (width 0.2) (layer "F.Cu") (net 11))
 (segment (start 64.77 91.44) (end 67.83 94.5) (width 0.2) (layer "F.Cu") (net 11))
 (segment (start 74.5 105.50851) (end 78.59186 109.60037) (width 0.2) (layer "F.Cu") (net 11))
 (segment (start 62.23 91.44) (end 63.293 90.377) (width 0.2) (layer "F.Cu") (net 5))
 (segment (start 77.025616 90.4875) (end 78.58125 90.4875) (width 0.2) (layer "F.Cu") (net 5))
 (segment (start 74.609116 92.904) (end 77.025616 90.4875) (width 0.2) (layer "F.Cu") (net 5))
 (segment (start 63.293 90.377) (end 65.62431 90.377) (width 0.2) (layer "F.Cu") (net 5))
 (segment (start 66.247 90.99969) (end 66.247 91.88031) (width 0.2) (layer "F.Cu") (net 5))
 (segment (start 66.247 91.88031) (end 67.27069 92.904) (width 0.2) (layer "F.Cu") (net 5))
 (segment (start 65.62431 90.377) (end 66.247 90.99969) (width 0.2) (layer "F.Cu") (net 5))
 (segment (start 67.27069 92.904) (end 74.609116 92.904) (width 0.2) (layer "F.Cu") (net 5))
 (segment (start 65.531999 75.438001) (end 65.531999 53.921999) (width 0.2) (layer "F.Cu") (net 3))
 (segment (start 65.531999 53.921999) (end 64 52.39) (width 0.2) (layer "F.Cu") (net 3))
 (segment (start 64.77 76.2) (end 65.531999 75.438001) (width 0.2) (layer "F.Cu") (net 3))
 (segment (start 69.85 76.2) (end 69.85 75.365) (width 0.2) (layer "F.Cu") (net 17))
 (segment (start 52.5365 43.4635) (end 52.5 43.5) (width 0.2) (layer "F.Cu") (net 4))
 (segment (start 62.002 111.51) (end 62.26 111.51) (width 0.2) (layer "F.Cu") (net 4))
 (segment (start 52.489853 84.989853) (end 52.489853 67) (width 0.2) (layer "F.Cu") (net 4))
 (segment (start 57.59031 92.503) (end 58.627 91.46631) (width 0.2) (layer "F.Cu") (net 4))
 (segment (start 64 50.64) (end 64 43.4635) (width 0.2) (layer "F.Cu") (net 4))
 (segment (start 52.5 56.457) (end 59.399 63.356) (width 0.2) (layer "F.Cu") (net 4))
 (segment (start 65.101 61.981) (end 64 60.88) (width 0.2) (layer "F.Cu") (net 4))
 (segment (start 52.5 66.989853) (end 52.489853 67) (width 0.2) (layer "F.Cu") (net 4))
 (segment (start 59.399 63.356) (end 61.5 63.356) (width 0.2) (layer "F.Cu") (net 4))
 (segment (start 61.5 63.38) (end 60.88 64) (width 0.2) (layer "F.Cu") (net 4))
 (segment (start 64 43.4635) (end 52.5365 43.4635) (width 0.2) (layer "F.Cu") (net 4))
 (segment (start 62.26 111.51) (end 64 113.25) (width 0.2) (layer "F.Cu") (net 4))
 (segment (start 64 103.01) (end 62.002 105.008) (width 0.2) (layer "F.Cu") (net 4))
 (segment (start 65.101 63.399) (end 65.101 61.981) (width 0.2) (layer "F.Cu") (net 4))
 (segment (start 52.5 64) (end 52.5 66.989853) (width 0.2) (layer "F.Cu") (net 4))
 (segment (start 63.17 103.01) (end 64 103.01) (width 0.2) (layer "F.Cu") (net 4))
 (segment (start 54.61 91.44) (end 55.673 92.503) (width 0.2) (layer "F.Cu") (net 4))
 (segment (start 60.88 64) (end 52.5 64) (width 0.2) (layer "F.Cu") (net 4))
 (segment (start 64 103.01) (end 64 100.83) (width 0.2) (layer "F.Cu") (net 4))
 (segment (start 52.5 86) (end 52.5 85) (width 0.2) (layer "F.Cu") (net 4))
 (segment (start 61.5 63.356) (end 61.524 63.356) (width 0.2) (layer "F.Cu") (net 4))
 (segment (start 52.5 85) (end 52.489853 84.989853) (width 0.2) (layer "F.Cu") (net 4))
 (segment (start 64.5 64) (end 65.101 63.399) (width 0.2) (layer "F.Cu") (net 4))
 (segment (start 61.5 63.356) (end 61.5 63.38) (width 0.2) (layer "F.Cu") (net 4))
 (segment (start 58.627 91.46631) (end 58.627 86) (width 0.2) (layer "F.Cu") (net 4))
 (segment (start 52.5 43.5) (end 52.5 56.457) (width 0.2) (layer "F.Cu") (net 4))
 (segment (start 64 100.83) (end 54.61 91.44) (width 0.2) (layer "F.Cu") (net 4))
 (segment (start 60.88 64) (end 64.5 64) (width 0.2) (layer "F.Cu") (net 4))
 (segment (start 58.627 86) (end 52.5 86) (width 0.2) (layer "F.Cu") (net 4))
 (segment (start 55.673 92.503) (end 57.59031 92.503) (width 0.2) (layer "F.Cu") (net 4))
 (segment (start 62.002 105.008) (end 62.002 111.51) (width 0.2) (layer "F.Cu") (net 4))
 (segment (start 58.401 52.739) (end 60.5 50.64) (width 0.2) (layer "F.Cu") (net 1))
 (segment (start 64 62.63) (end 58.401 57.031) (width 0.2) (layer "F.Cu") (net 1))
 (segment (start 58.401 57.031) (end 58.401 52.739) (width 0.2) (layer "F.Cu") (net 1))
 (segment (start 61.5 114.01) (end 62.49 115) (width 0.2) (layer "F.Cu") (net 8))
 (segment (start 60.5 103.01) (end 61.601 104.111) (width 0.2) (layer "F.Cu") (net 8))
 (segment (start 61.601 113.909) (end 61.5 114.01) (width 0.2) (layer "F.Cu") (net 8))
 (segment (start 62.49 115) (end 64 115) (width 0.2) (layer "F.Cu") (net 8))
 (segment (start 61.601 104.111) (end 61.601 113.909) (width 0.2) (layer "F.Cu") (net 8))
 (segment (start 64 104.76) (end 66 102.76) (width 0.2) (layer "F.Cu") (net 9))
 (segment (start 61 94) (end 61 83.5) (width 0.2) (layer "F.Cu") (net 9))
 (segment (start 60.5 83) (end 60.51 83) (width 0.2) (layer "F.Cu") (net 9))
 (segment (start 66 102.76) (end 66 99) (width 0.2) (layer "F.Cu") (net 9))
 (segment (start 66 99) (end 61 94) (width 0.2) (layer "F.Cu") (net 9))
 (segment (start 61 83.5) (end 60.5 83) (width 0.2) (layer "F.Cu") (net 9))
 (segment (start 60.51 83) (end 67.31 76.2) (width 0.2) (layer "F.Cu") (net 9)))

